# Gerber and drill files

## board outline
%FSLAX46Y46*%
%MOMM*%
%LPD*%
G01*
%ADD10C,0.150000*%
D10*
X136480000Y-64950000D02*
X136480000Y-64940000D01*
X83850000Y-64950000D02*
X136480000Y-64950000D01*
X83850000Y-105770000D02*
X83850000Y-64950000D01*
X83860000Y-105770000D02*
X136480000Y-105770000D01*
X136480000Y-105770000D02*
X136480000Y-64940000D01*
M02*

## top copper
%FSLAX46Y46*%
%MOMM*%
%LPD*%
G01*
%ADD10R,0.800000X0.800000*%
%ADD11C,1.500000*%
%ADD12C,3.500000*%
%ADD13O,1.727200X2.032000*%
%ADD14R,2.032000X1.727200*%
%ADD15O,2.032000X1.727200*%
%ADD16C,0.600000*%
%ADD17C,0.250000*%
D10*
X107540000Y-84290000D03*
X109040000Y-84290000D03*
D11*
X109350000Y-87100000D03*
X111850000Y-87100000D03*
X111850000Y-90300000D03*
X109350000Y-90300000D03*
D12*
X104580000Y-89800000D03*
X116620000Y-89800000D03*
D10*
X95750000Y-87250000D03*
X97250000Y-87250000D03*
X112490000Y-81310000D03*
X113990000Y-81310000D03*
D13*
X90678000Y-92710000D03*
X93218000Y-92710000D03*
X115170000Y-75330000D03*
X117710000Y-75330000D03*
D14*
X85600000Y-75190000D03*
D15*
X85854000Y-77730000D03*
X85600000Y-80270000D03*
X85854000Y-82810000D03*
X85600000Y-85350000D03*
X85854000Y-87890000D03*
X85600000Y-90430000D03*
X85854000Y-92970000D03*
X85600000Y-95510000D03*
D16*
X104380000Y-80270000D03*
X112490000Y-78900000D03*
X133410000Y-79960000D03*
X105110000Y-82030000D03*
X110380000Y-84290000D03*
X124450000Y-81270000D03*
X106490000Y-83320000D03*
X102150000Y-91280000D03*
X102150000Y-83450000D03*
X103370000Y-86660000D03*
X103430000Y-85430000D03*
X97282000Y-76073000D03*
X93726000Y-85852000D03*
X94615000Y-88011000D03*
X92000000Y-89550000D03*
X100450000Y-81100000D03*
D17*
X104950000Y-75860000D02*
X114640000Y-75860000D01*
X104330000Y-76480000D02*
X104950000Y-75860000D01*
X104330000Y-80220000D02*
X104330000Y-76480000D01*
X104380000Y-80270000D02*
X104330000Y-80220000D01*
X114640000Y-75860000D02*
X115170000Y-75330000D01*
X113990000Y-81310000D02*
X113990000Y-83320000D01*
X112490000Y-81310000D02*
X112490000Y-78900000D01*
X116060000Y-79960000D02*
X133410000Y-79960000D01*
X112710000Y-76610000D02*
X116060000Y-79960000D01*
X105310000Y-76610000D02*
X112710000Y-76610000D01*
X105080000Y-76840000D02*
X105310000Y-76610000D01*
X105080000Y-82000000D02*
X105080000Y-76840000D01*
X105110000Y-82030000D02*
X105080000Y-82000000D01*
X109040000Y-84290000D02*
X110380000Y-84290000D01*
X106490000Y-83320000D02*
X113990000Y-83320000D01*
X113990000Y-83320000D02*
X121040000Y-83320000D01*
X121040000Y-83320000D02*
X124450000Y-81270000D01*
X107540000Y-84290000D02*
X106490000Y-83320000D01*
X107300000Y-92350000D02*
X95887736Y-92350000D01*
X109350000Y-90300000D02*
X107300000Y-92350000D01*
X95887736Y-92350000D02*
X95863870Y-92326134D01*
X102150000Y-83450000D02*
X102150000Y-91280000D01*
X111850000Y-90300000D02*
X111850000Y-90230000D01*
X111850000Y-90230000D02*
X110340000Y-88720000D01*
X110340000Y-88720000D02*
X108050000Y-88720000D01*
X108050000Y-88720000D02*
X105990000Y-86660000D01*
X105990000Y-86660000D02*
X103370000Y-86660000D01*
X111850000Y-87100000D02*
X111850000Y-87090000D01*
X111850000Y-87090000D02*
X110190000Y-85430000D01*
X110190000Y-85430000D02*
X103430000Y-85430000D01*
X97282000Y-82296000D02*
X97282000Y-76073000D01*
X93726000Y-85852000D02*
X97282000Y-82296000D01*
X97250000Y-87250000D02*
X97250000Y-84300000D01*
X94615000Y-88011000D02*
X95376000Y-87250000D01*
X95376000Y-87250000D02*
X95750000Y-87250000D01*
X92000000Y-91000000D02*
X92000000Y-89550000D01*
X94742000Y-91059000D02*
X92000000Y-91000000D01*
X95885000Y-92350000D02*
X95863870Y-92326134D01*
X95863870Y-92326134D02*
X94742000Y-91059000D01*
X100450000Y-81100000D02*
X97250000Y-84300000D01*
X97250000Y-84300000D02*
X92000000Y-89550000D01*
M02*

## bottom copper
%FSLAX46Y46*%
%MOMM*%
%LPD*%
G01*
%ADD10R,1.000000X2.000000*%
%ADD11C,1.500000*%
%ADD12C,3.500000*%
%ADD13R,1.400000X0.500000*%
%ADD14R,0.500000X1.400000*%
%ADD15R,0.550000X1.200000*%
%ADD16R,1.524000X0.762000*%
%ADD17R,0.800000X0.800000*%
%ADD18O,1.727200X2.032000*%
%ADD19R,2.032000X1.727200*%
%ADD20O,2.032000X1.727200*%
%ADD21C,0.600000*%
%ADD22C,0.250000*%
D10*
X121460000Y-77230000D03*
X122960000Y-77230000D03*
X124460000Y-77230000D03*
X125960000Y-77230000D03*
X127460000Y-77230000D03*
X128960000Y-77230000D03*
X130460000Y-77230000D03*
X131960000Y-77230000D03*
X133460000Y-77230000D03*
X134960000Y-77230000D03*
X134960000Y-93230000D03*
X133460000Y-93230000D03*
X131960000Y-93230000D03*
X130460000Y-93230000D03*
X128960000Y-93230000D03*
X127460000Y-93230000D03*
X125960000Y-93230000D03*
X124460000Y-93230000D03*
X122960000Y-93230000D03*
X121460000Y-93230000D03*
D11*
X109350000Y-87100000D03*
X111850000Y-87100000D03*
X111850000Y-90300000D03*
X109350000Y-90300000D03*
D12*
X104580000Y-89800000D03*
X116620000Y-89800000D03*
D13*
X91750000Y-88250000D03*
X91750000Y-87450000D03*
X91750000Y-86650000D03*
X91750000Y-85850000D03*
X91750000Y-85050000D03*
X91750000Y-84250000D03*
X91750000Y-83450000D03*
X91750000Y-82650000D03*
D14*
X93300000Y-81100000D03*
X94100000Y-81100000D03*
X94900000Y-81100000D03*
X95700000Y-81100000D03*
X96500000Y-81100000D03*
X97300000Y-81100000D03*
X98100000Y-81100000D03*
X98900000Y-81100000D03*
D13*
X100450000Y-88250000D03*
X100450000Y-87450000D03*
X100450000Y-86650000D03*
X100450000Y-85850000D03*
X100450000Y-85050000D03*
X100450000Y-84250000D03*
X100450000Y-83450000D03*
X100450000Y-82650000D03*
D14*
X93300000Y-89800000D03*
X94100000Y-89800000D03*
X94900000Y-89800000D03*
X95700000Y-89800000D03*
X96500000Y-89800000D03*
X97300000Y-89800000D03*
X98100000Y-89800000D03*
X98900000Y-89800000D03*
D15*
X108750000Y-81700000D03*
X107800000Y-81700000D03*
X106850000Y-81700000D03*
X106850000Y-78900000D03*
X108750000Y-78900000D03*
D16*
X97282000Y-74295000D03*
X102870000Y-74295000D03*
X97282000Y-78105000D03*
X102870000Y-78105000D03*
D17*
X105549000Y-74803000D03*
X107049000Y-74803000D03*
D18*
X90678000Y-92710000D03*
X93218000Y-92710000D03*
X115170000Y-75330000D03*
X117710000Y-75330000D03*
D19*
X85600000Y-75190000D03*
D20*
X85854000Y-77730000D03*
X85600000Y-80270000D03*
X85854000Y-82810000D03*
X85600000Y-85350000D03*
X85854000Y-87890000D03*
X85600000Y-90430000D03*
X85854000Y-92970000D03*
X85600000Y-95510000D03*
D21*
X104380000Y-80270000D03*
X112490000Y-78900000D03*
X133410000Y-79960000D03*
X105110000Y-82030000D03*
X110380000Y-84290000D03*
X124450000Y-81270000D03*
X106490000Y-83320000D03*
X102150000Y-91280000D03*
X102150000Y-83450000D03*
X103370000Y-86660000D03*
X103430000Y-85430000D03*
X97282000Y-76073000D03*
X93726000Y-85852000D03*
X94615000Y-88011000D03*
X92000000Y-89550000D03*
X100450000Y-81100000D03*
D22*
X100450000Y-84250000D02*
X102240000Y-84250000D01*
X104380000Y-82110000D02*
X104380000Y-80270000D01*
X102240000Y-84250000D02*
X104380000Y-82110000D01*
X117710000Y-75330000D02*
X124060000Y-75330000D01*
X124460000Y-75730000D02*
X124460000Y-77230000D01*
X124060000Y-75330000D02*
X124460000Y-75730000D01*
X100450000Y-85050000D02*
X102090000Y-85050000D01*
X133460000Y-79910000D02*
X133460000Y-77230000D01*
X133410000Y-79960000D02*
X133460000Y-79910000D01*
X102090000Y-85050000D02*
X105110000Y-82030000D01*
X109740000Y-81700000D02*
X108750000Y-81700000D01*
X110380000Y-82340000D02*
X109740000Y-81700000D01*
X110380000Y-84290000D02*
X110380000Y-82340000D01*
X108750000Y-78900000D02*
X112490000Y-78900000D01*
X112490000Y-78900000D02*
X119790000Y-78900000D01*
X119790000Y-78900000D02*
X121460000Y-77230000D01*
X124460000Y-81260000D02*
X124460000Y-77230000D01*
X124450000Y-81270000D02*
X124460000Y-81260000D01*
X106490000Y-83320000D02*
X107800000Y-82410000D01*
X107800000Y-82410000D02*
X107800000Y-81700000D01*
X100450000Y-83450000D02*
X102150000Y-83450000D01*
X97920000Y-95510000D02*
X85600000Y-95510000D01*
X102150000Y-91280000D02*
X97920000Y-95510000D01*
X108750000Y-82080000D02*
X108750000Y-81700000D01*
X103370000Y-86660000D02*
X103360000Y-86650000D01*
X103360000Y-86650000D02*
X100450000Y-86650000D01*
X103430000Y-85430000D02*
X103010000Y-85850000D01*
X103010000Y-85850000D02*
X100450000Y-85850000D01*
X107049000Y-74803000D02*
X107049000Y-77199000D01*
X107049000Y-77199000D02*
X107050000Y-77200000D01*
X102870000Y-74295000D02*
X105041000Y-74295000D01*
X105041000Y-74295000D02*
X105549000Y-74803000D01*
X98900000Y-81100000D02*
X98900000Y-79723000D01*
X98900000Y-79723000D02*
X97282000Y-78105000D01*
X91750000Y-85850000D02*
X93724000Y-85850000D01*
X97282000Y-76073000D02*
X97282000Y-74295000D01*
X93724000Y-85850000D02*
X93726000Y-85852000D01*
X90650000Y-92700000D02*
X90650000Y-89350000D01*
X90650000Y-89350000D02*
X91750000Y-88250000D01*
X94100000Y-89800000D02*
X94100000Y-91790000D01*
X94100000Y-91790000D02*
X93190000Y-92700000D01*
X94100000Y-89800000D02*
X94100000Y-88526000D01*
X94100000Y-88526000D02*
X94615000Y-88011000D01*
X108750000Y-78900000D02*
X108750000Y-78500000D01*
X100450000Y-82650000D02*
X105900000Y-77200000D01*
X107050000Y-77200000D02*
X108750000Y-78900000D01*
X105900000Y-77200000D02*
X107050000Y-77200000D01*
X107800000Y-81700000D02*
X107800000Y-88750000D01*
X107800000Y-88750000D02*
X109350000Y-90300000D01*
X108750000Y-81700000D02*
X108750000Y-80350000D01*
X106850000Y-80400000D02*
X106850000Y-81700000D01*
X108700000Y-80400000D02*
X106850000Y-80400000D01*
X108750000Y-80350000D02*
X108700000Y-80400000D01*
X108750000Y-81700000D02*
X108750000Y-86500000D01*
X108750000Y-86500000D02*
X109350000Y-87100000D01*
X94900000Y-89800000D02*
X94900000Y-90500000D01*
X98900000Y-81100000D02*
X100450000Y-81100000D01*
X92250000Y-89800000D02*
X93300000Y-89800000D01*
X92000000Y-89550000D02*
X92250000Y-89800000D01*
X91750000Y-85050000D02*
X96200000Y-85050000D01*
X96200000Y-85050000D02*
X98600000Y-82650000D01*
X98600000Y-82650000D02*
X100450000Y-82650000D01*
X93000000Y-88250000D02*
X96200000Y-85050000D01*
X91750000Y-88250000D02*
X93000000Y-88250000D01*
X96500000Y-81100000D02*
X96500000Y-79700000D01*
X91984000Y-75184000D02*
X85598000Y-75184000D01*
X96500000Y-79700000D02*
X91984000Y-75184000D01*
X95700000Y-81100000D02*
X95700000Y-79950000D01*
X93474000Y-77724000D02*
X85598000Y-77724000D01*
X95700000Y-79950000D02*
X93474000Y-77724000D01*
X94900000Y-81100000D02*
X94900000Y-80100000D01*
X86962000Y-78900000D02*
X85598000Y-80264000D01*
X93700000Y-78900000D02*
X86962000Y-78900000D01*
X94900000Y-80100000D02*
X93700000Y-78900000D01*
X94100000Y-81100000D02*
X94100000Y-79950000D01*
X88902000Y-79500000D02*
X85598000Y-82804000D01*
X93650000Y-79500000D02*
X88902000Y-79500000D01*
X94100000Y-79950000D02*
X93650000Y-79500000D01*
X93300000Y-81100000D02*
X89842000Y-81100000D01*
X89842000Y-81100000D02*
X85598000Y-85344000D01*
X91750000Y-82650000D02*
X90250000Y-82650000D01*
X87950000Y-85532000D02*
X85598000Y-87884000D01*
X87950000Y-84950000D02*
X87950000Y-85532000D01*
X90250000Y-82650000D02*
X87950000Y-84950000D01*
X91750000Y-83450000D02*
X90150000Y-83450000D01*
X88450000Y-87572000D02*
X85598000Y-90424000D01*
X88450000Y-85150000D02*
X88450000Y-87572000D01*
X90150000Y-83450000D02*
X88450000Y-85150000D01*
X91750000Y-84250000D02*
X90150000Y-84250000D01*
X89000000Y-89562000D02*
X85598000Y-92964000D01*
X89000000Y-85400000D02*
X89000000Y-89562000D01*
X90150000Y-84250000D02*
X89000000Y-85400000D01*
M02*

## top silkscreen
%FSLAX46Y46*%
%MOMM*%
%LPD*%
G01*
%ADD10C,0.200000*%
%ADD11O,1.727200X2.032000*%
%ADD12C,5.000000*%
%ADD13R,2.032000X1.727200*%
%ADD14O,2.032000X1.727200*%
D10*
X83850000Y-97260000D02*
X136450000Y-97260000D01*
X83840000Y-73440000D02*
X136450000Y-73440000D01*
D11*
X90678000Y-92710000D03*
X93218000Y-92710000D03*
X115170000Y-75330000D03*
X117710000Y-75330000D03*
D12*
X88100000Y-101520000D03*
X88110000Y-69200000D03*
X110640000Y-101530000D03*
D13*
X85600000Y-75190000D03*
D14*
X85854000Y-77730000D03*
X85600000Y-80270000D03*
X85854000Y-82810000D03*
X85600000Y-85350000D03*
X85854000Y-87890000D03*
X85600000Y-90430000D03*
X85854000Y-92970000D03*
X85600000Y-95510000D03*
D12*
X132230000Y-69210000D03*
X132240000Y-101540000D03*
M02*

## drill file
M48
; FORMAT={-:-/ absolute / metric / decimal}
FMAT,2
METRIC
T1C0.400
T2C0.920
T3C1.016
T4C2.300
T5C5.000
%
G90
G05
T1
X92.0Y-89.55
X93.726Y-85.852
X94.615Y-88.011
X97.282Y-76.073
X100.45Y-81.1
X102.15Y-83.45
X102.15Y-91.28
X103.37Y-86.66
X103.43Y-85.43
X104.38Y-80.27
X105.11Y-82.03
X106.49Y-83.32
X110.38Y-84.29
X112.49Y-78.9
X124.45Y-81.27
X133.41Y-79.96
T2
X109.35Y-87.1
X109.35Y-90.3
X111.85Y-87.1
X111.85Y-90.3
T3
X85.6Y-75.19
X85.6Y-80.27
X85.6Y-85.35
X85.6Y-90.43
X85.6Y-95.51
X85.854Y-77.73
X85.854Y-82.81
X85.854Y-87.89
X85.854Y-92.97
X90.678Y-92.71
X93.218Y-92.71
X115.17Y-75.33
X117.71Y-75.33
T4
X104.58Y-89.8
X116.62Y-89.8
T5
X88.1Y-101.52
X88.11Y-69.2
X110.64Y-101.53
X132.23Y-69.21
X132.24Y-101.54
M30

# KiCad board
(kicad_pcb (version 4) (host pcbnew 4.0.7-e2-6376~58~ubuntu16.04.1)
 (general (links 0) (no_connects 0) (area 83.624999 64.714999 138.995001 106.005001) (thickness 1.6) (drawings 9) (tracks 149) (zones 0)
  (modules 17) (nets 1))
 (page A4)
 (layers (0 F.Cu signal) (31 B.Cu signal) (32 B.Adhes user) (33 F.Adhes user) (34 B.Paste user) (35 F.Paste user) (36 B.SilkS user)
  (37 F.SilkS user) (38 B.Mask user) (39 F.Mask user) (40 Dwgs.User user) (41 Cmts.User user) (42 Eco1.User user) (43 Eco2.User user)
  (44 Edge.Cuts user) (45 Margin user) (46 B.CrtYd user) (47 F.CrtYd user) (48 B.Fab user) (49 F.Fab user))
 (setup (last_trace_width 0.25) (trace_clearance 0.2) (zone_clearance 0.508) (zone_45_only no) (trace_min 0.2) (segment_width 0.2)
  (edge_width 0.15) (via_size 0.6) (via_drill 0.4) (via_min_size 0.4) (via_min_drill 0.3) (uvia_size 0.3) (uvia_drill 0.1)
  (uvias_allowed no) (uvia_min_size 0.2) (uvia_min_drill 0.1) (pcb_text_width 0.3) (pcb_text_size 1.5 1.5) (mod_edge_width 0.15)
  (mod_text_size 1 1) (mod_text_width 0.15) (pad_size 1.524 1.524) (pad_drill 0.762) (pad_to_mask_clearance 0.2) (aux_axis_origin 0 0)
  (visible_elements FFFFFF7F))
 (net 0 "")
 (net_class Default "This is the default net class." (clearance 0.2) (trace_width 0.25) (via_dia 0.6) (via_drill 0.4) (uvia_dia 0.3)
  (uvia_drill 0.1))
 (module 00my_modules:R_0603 (layer F.Cu) (at 108.29 84.29)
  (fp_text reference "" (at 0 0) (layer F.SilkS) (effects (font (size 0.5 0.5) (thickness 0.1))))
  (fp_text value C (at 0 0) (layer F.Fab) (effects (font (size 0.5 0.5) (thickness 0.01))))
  (pad 1 smd rect (at -0.75 0) (size 0.8 0.8) (layers F.Cu F.Paste F.Mask))
  (pad 2 smd rect (at 0.75 0) (size 0.8 0.8) (layers F.Cu F.Paste F.Mask)))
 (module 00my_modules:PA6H (layer B.Cu) (at 128.21 85.23 270)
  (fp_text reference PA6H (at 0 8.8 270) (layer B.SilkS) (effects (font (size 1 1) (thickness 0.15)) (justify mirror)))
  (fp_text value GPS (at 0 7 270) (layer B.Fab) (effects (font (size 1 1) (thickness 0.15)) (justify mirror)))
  (pad VCC smd rect (at -8 6.75 270) (size 2 1) (layers B.Cu B.Paste B.Mask))
  (pad 2 smd rect (at -8 5.25 270) (size 2 1) (layers B.Cu B.Paste B.Mask))
  (pad GND smd rect (at -8 3.75 270) (size 2 1) (layers B.Cu B.Paste B.Mask))
  (pad 4 smd rect (at -8 2.25 270) (size 2 1) (layers B.Cu B.Paste B.Mask))
  (pad 5 smd rect (at -8 0.75 270) (size 2 1) (layers B.Cu B.Paste B.Mask))
  (pad 6 smd rect (at -8 -0.75 270) (size 2 1) (layers B.Cu B.Paste B.Mask))
  (pad 7 smd rect (at -8 -2.25 270) (size 2 1) (layers B.Cu B.Paste B.Mask))
  (pad 8 smd rect (at -8 -3.75 270) (size 2 1) (layers B.Cu B.Paste B.Mask))
  (pad TX smd rect (at -8 -5.25 270) (size 2 1) (layers B.Cu B.Paste B.Mask))
  (pad RX smd rect (at -8 -6.75 270) (size 2 1) (layers B.Cu B.Paste B.Mask))
  (pad 11 smd rect (at 8 -6.75 270) (size 2 1) (layers B.Cu B.Paste B.Mask))
  (pad 12 smd rect (at 8 -5.25 270) (size 2 1) (layers B.Cu B.Paste B.Mask))
  (pad 13 smd rect (at 8 -3.75 270) (size 2 1) (layers B.Cu B.Paste B.Mask))
  (pad 14 smd rect (at 8 -2.25 270) (size 2 1) (layers B.Cu B.Paste B.Mask))
  (pad 15 smd rect (at 8 -0.75 270) (size 2 1) (layers B.Cu B.Paste B.Mask))
  (pad 16 smd rect (at 8 0.75 270) (size 2 1) (layers B.Cu B.Paste B.Mask))
  (pad 17 smd rect (at 8 2.25 270) (size 2 1) (layers B.Cu B.Paste B.Mask))
  (pad 18 smd rect (at 8 3.75 270) (size 2 1) (layers B.Cu B.Paste B.Mask))
  (pad 19 smd rect (at 8 5.25 270) (size 2 1) (layers B.Cu B.Paste B.Mask))
  (pad 20 smd rect (at 8 6.75 270) (size 2 1) (layers B.Cu B.Paste B.Mask)))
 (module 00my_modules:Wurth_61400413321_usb (layer B.Cu) (at 110.6 89.8 180)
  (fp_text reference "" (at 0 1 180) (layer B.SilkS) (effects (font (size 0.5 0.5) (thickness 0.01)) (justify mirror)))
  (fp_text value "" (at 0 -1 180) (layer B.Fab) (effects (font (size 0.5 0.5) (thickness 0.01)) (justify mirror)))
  (pad V thru_hole circle (at 1.25 2.7 180) (size 1.5 1.5) (drill 0.92) (layers *.Cu *.Mask B.SilkS))
  (pad - thru_hole circle (at -1.25 2.7 180) (size 1.5 1.5) (drill 0.92) (layers *.Cu *.Mask B.SilkS))
  (pad + thru_hole circle (at -1.25 -0.5 180) (size 1.5 1.5) (drill 0.92) (layers *.Cu *.Mask B.SilkS))
  (pad G thru_hole circle (at 1.25 -0.5 180) (size 1.5 1.5) (drill 0.92) (layers *.Cu *.Mask B.SilkS))
  (pad X thru_hole circle (at 6.02 0 180) (size 3.5 3.5) (drill 2.3) (layers *.Cu *.Mask B.SilkS))
  (pad X thru_hole circle (at -6.02 0 180) (size 3.5 3.5) (drill 2.3) (layers *.Cu *.Mask B.SilkS)))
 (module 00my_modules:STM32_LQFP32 (layer B.Cu) (at 96.1 85.45)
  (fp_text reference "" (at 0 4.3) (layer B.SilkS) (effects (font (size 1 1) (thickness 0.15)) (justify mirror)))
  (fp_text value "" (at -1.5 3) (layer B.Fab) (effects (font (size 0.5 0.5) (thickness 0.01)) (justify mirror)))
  (pad 3.3 smd rect (at -4.35 2.8) (size 1.4 0.5) (layers B.Cu B.Paste B.Mask))
  (pad PF0 smd rect (at -4.35 2) (size 1.4 0.5) (layers B.Cu B.Paste B.Mask))
  (pad PF1 smd rect (at -4.35 1.2) (size 1.4 0.5) (layers B.Cu B.Paste B.Mask))
  (pad RST smd rect (at -4.35 0.4) (size 1.4 0.5) (layers B.Cu B.Paste B.Mask))
  (pad 3.3 smd rect (at -4.35 -0.4) (size 1.4 0.5) (layers B.Cu B.Paste B.Mask))
  (pad PA0 smd rect (at -4.35 -1.2) (size 1.4 0.5) (layers B.Cu B.Paste B.Mask))
  (pad PA1 smd rect (at -4.35 -2) (size 1.4 0.5) (layers B.Cu B.Paste B.Mask))
  (pad PA2 smd rect (at -4.35 -2.8) (size 1.4 0.5) (layers B.Cu B.Paste B.Mask))
  (pad PA3 smd rect (at -2.8 -4.35 270) (size 1.4 0.5) (layers B.Cu B.Paste B.Mask))
  (pad PA4 smd rect (at -2 -4.35 270) (size 1.4 0.5) (layers B.Cu B.Paste B.Mask))
  (pad PA5 smd rect (at -1.2 -4.35 270) (size 1.4 0.5) (layers B.Cu B.Paste B.Mask))
  (pad PA6 smd rect (at -0.4 -4.35 270) (size 1.4 0.5) (layers B.Cu B.Paste B.Mask))
  (pad PA7 smd rect (at 0.4 -4.35 270) (size 1.4 0.5) (layers B.Cu B.Paste B.Mask))
  (pad PB0 smd rect (at 1.2 -4.35 270) (size 1.4 0.5) (layers B.Cu B.Paste B.Mask))
  (pad PB1 smd rect (at 2 -4.35 270) (size 1.4 0.5) (layers B.Cu B.Paste B.Mask))
  (pad GND smd rect (at 2.8 -4.35 270) (size 1.4 0.5) (layers B.Cu B.Paste B.Mask))
  (pad PA14 smd rect (at 4.35 2.8) (size 1.4 0.5) (layers B.Cu B.Paste B.Mask))
  (pad PA13 smd rect (at 4.35 2) (size 1.4 0.5) (layers B.Cu B.Paste B.Mask))
  (pad PA12 smd rect (at 4.35 1.2) (size 1.4 0.5) (layers B.Cu B.Paste B.Mask))
  (pad PA11 smd rect (at 4.35 0.4) (size 1.4 0.5) (layers B.Cu B.Paste B.Mask))
  (pad PA10 smd rect (at 4.35 -0.4) (size 1.4 0.5) (layers B.Cu B.Paste B.Mask))
  (pad PA9 smd rect (at 4.35 -1.2) (size 1.4 0.5) (layers B.Cu B.Paste B.Mask))
  (pad PA8 smd rect (at 4.35 -2) (size 1.4 0.5) (layers B.Cu B.Paste B.Mask))
  (pad 3.3 smd rect (at 4.35 -2.8) (size 1.4 0.5) (layers B.Cu B.Paste B.Mask))
  (pad GND smd rect (at -2.8 4.35 270) (size 1.4 0.5) (layers B.Cu B.Paste B.Mask))
  (pad BOOT smd rect (at -2 4.35 270) (size 1.4 0.5) (layers B.Cu B.Paste B.Mask))
  (pad PB7 smd rect (at -1.2 4.35 270) (size 1.4 0.5) (layers B.Cu B.Paste B.Mask))
  (pad PB6 smd rect (at -0.4 4.35 270) (size 1.4 0.5) (layers B.Cu B.Paste B.Mask))
  (pad PB5 smd rect (at 0.4 4.35 270) (size 1.4 0.5) (layers B.Cu B.Paste B.Mask))
  (pad PB4 smd rect (at 1.2 4.35 270) (size 1.4 0.5) (layers B.Cu B.Paste B.Mask))
  (pad PB3 smd rect (at 2 4.35 270) (size 1.4 0.5) (layers B.Cu B.Paste B.Mask))
  (pad PA15 smd rect (at 2.8 4.35 270) (size 1.4 0.5) (layers B.Cu B.Paste B.Mask)))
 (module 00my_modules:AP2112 (layer B.Cu) (at 107.8 80.3 90)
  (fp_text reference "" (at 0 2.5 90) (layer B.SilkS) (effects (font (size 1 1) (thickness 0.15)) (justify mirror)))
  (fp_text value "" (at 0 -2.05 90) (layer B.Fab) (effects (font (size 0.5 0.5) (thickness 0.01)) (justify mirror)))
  (pad VIN smd rect (at -1.4 0.95 90) (size 1.2 0.55) (layers B.Cu B.Paste B.Mask))
  (pad GND smd rect (at -1.4 0 90) (size 1.2 0.55) (layers B.Cu B.Paste B.Mask))
  (pad EN smd rect (at -1.4 -0.95 90) (size 1.2 0.55) (layers B.Cu B.Paste B.Mask))
  (pad NC smd rect (at 1.4 -0.95 90) (size 1.2 0.55) (layers B.Cu B.Paste B.Mask))
  (pad VOUT smd rect (at 1.4 0.95 90) (size 1.2 0.55) (layers B.Cu B.Paste B.Mask)))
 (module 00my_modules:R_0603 (layer F.Cu) (at 96.5 87.25)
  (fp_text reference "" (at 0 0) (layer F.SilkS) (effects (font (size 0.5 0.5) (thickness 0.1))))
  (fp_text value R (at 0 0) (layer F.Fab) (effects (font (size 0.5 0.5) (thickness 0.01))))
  (pad 1 smd rect (at -0.75 0) (size 0.8 0.8) (layers F.Cu F.Paste F.Mask))
  (pad 2 smd rect (at 0.75 0) (size 0.8 0.8) (layers F.Cu F.Paste F.Mask)))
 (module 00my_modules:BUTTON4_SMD (layer B.Cu) (at 100.076 76.2)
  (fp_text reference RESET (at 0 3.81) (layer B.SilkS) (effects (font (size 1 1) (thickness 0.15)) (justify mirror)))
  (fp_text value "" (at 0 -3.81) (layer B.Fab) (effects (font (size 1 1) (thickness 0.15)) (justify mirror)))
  (pad 1 smd rect (at -2.794 -1.905) (size 1.524 0.762) (layers B.Cu B.Paste B.Mask))
  (pad 2 smd rect (at 2.794 -1.905) (size 1.524 0.762) (layers B.Cu B.Paste B.Mask))
  (pad 3 smd rect (at -2.794 1.905) (size 1.524 0.762) (layers B.Cu B.Paste B.Mask))
  (pad 4 smd rect (at 2.794 1.905) (size 1.524 0.762) (layers B.Cu B.Paste B.Mask)))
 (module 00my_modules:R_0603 (layer B.Cu) (at 106.299 74.803)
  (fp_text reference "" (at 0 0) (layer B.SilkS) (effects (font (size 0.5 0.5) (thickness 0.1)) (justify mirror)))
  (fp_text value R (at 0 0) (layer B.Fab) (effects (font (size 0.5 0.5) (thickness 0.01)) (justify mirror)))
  (pad 1 smd rect (at -0.75 0) (size 0.8 0.8) (layers B.Cu B.Paste B.Mask))
  (pad 2 smd rect (at 0.75 0) (size 0.8 0.8) (layers B.Cu B.Paste B.Mask)))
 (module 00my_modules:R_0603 (layer F.Cu) (at 113.24 81.31)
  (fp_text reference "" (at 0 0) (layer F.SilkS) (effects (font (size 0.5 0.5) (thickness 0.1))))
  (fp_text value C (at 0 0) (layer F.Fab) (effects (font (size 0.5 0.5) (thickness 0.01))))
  (pad 1 smd rect (at -0.75 0) (size 0.8 0.8) (layers F.Cu F.Paste F.Mask))
  (pad 2 smd rect (at 0.75 0) (size 0.8 0.8) (layers F.Cu F.Paste F.Mask)))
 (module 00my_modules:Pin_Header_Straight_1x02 (layer F.Cu) (at 90.678 92.71 90)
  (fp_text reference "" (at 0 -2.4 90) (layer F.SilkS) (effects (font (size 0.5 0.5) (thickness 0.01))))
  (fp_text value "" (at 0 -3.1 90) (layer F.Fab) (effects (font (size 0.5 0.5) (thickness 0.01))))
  (pad 1 thru_hole oval (at 0 0 90) (size 2.032 1.7272) (drill 1.016) (layers *.Cu *.Mask F.SilkS))
  (pad 2 thru_hole oval (at 0 2.54 90) (size 2.032 1.7272) (drill 1.016) (layers *.Cu *.Mask F.SilkS)))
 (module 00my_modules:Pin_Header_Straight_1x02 (layer F.Cu) (at 115.17 75.33 90)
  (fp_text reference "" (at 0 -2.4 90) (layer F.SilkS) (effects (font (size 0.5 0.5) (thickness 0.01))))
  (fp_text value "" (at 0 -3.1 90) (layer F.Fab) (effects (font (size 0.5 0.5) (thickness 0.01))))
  (pad 1 thru_hole oval (at 0 0 90) (size 2.032 1.7272) (drill 1.016) (layers *.Cu *.Mask F.SilkS))
  (pad 2 thru_hole oval (at 0 2.54 90) (size 2.032 1.7272) (drill 1.016) (layers *.Cu *.Mask F.SilkS)))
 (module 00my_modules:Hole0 (layer F.Cu) (at 88.1 101.52)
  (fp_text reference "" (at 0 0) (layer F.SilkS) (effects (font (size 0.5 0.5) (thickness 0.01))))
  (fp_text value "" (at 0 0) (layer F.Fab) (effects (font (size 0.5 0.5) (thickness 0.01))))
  (pad "" np_thru_hole circle (at 0 0) (size 5 5) (drill 5) (layers *.Cu *.Mask F.SilkS)))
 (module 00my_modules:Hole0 (layer F.Cu) (at 88.11 69.2)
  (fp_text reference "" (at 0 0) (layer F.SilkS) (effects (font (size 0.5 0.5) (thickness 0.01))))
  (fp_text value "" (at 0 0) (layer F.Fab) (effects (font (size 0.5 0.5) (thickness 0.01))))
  (pad "" np_thru_hole circle (at 0 0) (size 5 5) (drill 5) (layers *.Cu *.Mask F.SilkS)))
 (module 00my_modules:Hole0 (layer F.Cu) (at 110.64 101.53)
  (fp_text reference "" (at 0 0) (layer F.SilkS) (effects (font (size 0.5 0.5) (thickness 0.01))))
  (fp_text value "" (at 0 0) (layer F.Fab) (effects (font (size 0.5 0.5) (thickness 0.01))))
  (pad "" np_thru_hole circle (at 0 0) (size 5 5) (drill 5) (layers *.Cu *.Mask F.SilkS)))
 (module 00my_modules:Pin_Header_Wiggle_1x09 (layer F.Cu) (at 85.6 75.19)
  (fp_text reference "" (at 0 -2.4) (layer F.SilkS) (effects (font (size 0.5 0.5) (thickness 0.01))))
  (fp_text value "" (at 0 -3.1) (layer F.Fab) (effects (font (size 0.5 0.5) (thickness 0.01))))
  (pad 1 thru_hole rect (at 0 0) (size 2.032 1.7272) (drill 1.016) (layers *.Cu *.Mask F.SilkS))
  (pad 2 thru_hole oval (at 0.254 2.54) (size 2.032 1.7272) (drill 1.016) (layers *.Cu *.Mask F.SilkS))
  (pad 3 thru_hole oval (at 0 5.08) (size 2.032 1.7272) (drill 1.016) (layers *.Cu *.Mask F.SilkS))
  (pad 4 thru_hole oval (at 0.254 7.62) (size 2.032 1.7272) (drill 1.016) (layers *.Cu *.Mask F.SilkS))
  (pad 5 thru_hole oval (at 0 10.16) (size 2.032 1.7272) (drill 1.016) (layers *.Cu *.Mask F.SilkS))
  (pad 6 thru_hole oval (at 0.254 12.7) (size 2.032 1.7272) (drill 1.016) (layers *.Cu *.Mask F.SilkS))
  (pad 7 thru_hole oval (at 0 15.24) (size 2.032 1.7272) (drill 1.016) (layers *.Cu *.Mask F.SilkS))
  (pad 8 thru_hole oval (at 0.254 17.78) (size 2.032 1.7272) (drill 1.016) (layers *.Cu *.Mask F.SilkS))
  (pad 9 thru_hole oval (at 0 20.32) (size 2.032 1.7272) (drill 1.016) (layers *.Cu *.Mask F.SilkS)))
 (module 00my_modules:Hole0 (layer F.Cu) (at 132.23 69.21)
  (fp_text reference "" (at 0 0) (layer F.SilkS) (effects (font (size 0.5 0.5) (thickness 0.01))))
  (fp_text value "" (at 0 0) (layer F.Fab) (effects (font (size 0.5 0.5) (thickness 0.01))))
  (pad "" np_thru_hole circle (at 0 0) (size 5 5) (drill 5) (layers *.Cu *.Mask F.SilkS)))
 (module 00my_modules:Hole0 (layer F.Cu) (at 132.24 101.54)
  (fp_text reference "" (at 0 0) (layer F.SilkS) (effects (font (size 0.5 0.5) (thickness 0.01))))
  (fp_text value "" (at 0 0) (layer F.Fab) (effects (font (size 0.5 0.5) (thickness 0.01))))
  (pad "" np_thru_hole circle (at 0 0) (size 5 5) (drill 5) (layers *.Cu *.Mask F.SilkS)))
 (gr_line (start 83.85 97.26) (end 136.45 97.26) (angle 90) (layer F.SilkS) (width 0.2))
 (gr_line (start 83.84 73.44) (end 136.45 73.44) (angle 90) (layer F.SilkS) (width 0.2))
 (gr_line (start 136.48 64.95) (end 136.48 64.94) (angle 90) (layer Edge.Cuts) (width 0.15))
 (gr_line (start 83.85 64.95) (end 136.48 64.95) (angle 90) (layer Edge.Cuts) (width 0.15))
 (gr_line (start 83.85 105.77) (end 83.85 64.95) (angle 90) (layer Edge.Cuts) (width 0.15))
 (gr_line (start 83.86 105.77) (end 136.48 105.77) (angle 90) (layer Edge.Cuts) (width 0.15))
 (gr_line (start 136.48 105.77) (end 136.48 64.94) (angle 90) (layer Edge.Cuts) (width 0.15))
 (segment (start 100.45 84.25) (end 102.24 84.25) (width 0.25) (layer B.Cu) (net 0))
 (segment (start 104.95 75.86) (end 114.64 75.86) (width 0.25) (layer F.Cu) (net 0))
 (segment (start 104.33 76.48) (end 104.95 75.86) (width 0.25) (layer F.Cu) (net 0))
 (segment (start 104.33 80.22) (end 104.33 76.48) (width 0.25) (layer F.Cu) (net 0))
 (segment (start 104.38 80.27) (end 104.33 80.22) (width 0.25) (layer F.Cu) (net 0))
 (via (at 104.38 80.27) (size 0.6) (drill 0.4) (layers F.Cu B.Cu) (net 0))
 (segment (start 104.38 82.11) (end 104.38 80.27) (width 0.25) (layer B.Cu) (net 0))
 (segment (start 102.24 84.25) (end 104.38 82.11) (width 0.25) (layer B.Cu) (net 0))
 (segment (start 114.64 75.86) (end 115.17 75.33) (width 0.25) (layer F.Cu) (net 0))
 (segment (start 117.71 75.33) (end 124.06 75.33) (width 0.25) (layer B.Cu) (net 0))
 (segment (start 124.46 75.73) (end 124.46 77.23) (width 0.25) (layer B.Cu) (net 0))
 (segment (start 124.06 75.33) (end 124.46 75.73) (width 0.25) (layer B.Cu) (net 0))
 (segment (start 113.99 81.31) (end 113.99 83.32) (width 0.25) (layer F.Cu) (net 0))
 (segment (start 112.49 81.31) (end 112.49 78.9) (width 0.25) (layer F.Cu) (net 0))
 (via (at 112.49 78.9) (size 0.6) (drill 0.4) (layers F.Cu B.Cu) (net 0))
 (segment (start 100.45 85.05) (end 102.09 85.05) (width 0.25) (layer B.Cu) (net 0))
 (segment (start 133.46 79.91) (end 133.46 77.23) (width 0.25) (layer B.Cu) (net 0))
 (segment (start 133.41 79.96) (end 133.46 79.91) (width 0.25) (layer B.Cu) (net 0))
 (via (at 133.41 79.96) (size 0.6) (drill 0.4) (layers F.Cu B.Cu) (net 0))
 (segment (start 116.06 79.96) (end 133.41 79.96) (width 0.25) (layer F.Cu) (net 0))
 (segment (start 112.71 76.61) (end 116.06 79.96) (width 0.25) (layer F.Cu) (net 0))
 (segment (start 105.31 76.61) (end 112.71 76.61) (width 0.25) (layer F.Cu) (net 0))
 (segment (start 105.08 76.84) (end 105.31 76.61) (width 0.25) (layer F.Cu) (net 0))
 (segment (start 105.08 82) (end 105.08 76.84) (width 0.25) (layer F.Cu) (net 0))
 (segment (start 105.11 82.03) (end 105.08 82) (width 0.25) (layer F.Cu) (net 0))
 (via (at 105.11 82.03) (size 0.6) (drill 0.4) (layers F.Cu B.Cu) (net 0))
 (segment (start 102.09 85.05) (end 105.11 82.03) (width 0.25) (layer B.Cu) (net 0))
 (segment (start 109.04 84.29) (end 110.38 84.29) (width 0.25) (layer F.Cu) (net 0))
 (segment (start 109.74 81.7) (end 108.75 81.7) (width 0.25) (layer B.Cu) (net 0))
 (segment (start 110.38 82.34) (end 109.74 81.7) (width 0.25) (layer B.Cu) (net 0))
 (segment (start 110.38 84.29) (end 110.38 82.34) (width 0.25) (layer B.Cu) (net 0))
 (via (at 110.38 84.29) (size 0.6) (drill 0.4) (layers F.Cu B.Cu) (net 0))
 (segment (start 108.75 78.9) (end 112.49 78.9) (width 0.25) (layer B.Cu) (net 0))
 (segment (start 112.49 78.9) (end 119.79 78.9) (width 0.25) (layer B.Cu) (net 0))
 (segment (start 119.79 78.9) (end 121.46 77.23) (width 0.25) (layer B.Cu) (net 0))
 (segment (start 106.49 83.32) (end 113.99 83.32) (width 0.25) (layer F.Cu) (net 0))
 (segment (start 113.99 83.32) (end 121.04 83.32) (width 0.25) (layer F.Cu) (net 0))
 (segment (start 124.46 81.26) (end 124.46 77.23) (width 0.25) (layer B.Cu) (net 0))
 (segment (start 124.45 81.27) (end 124.46 81.26) (width 0.25) (layer B.Cu) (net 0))
 (via (at 124.45 81.27) (size 0.6) (drill 0.4) (layers F.Cu B.Cu) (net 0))
 (segment (start 121.04 83.32) (end 124.45 81.27) (width 0.25) (layer F.Cu) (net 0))
 (segment (start 107.54 84.29) (end 106.49 83.32) (width 0.25) (layer F.Cu) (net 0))
 (via (at 106.49 83.32) (size 0.6) (drill 0.4) (layers F.Cu B.Cu) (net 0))
 (segment (start 106.49 83.32) (end 107.8 82.41) (width 0.25) (layer B.Cu) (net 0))
 (segment (start 107.8 82.41) (end 107.8 81.7) (width 0.25) (layer B.Cu) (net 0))
 (segment (start 107.3 92.35) (end 95.887736 92.35) (width 0.25) (layer F.Cu) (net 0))
 (segment (start 109.35 90.3) (end 107.3 92.35) (width 0.25) (layer F.Cu) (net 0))
 (segment (start 95.887736 92.35) (end 95.86387 92.326134) (width 0.25) (layer F.Cu) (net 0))
 (segment (start 100.45 83.45) (end 102.15 83.45) (width 0.25) (layer B.Cu) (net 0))
 (segment (start 97.92 95.51) (end 85.6 95.51) (width 0.25) (layer B.Cu) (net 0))
 (segment (start 102.15 91.28) (end 97.92 95.51) (width 0.25) (layer B.Cu) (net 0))
 (via (at 102.15 91.28) (size 0.6) (drill 0.4) (layers F.Cu B.Cu) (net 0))
 (segment (start 102.15 83.45) (end 102.15 91.28) (width 0.25) (layer F.Cu) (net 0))
 (via (at 102.15 83.45) (size 0.6) (drill 0.4) (layers F.Cu B.Cu) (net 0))
 (segment (start 108.75 82.08) (end 108.75 81.7) (width 0.25) (layer B.Cu) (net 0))
 (segment (start 111.85 90.3) (end 111.85 90.23) (width 0.25) (layer F.Cu) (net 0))
 (segment (start 111.85 90.23) (end 110.34 88.72) (width 0.25) (layer F.Cu) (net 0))
 (segment (start 110.34 88.72) (end 108.05 88.72) (width 0.25) (layer F.Cu) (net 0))
 (segment (start 108.05 88.72) (end 105.99 86.66) (width 0.25) (layer F.Cu) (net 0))
 (segment (start 105.99 86.66) (end 103.37 86.66) (width 0.25) (layer F.Cu) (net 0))
 (via (at 103.37 86.66) (size 0.6) (drill 0.4) (layers F.Cu B.Cu) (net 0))
 (segment (start 103.37 86.66) (end 103.36 86.65) (width 0.25) (layer B.Cu) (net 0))
 (segment (start 103.36 86.65) (end 100.45 86.65) (width 0.25) (layer B.Cu) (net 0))
 (segment (start 111.85 87.1) (end 111.85 87.09) (width 0.25) (layer F.Cu) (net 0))
 (segment (start 111.85 87.09) (end 110.19 85.43) (width 0.25) (layer F.Cu) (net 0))
 (segment (start 110.19 85.43) (end 103.43 85.43) (width 0.25) (layer F.Cu) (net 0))
 (via (at 103.43 85.43) (size 0.6) (drill 0.4) (layers F.Cu B.Cu) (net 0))
 (segment (start 103.43 85.43) (end 103.01 85.85) (width 0.25) (layer B.Cu) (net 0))
 (segment (start 103.01 85.85) (end 100.45 85.85) (width 0.25) (layer B.Cu) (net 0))
 (segment (start 107.049 74.803) (end 107.049 77.199) (width 0.25) (layer B.Cu) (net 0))
 (segment (start 107.049 77.199) (end 107.05 77.2) (width 0.25) (layer B.Cu) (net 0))
 (segment (start 102.87 74.295) (end 105.041 74.295) (width 0.25) (layer B.Cu) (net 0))
 (segment (start 105.041 74.295) (end 105.549 74.803) (width 0.25) (layer B.Cu) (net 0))
 (segment (start 98.9 81.1) (end 98.9 79.723) (width 0.25) (layer B.Cu) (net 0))
 (segment (start 98.9 79.723) (end 97.282 78.105) (width 0.25) (layer B.Cu) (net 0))
 (segment (start 91.75 85.85) (end 93.724 85.85) (width 0.25) (layer B.Cu) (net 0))
 (segment (start 97.282 76.073) (end 97.282 74.295) (width 0.25) (layer B.Cu) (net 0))
 (via (at 97.282 76.073) (size 0.6) (drill 0.4) (layers F.Cu B.Cu) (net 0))
 (segment (start 97.282 82.296) (end 97.282 76.073) (width 0.25) (layer F.Cu) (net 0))
 (segment (start 93.726 85.852) (end 97.282 82.296) (width 0.25) (layer F.Cu) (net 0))
 (via (at 93.726 85.852) (size 0.6) (drill 0.4) (layers F.Cu B.Cu) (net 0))
 (segment (start 93.724 85.85) (end 93.726 85.852) (width 0.25) (layer B.Cu) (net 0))
 (segment (start 90.65 92.7) (end 90.65 89.35) (width 0.25) (layer B.Cu) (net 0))
 (segment (start 90.65 89.35) (end 91.75 88.25) (width 0.25) (layer B.Cu) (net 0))
 (segment (start 94.1 89.8) (end 94.1 91.79) (width 0.25) (layer B.Cu) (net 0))
 (segment (start 94.1 91.79) (end 93.19 92.7) (width 0.25) (layer B.Cu) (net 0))
 (segment (start 97.25 87.25) (end 97.25 84.3) (width 0.25) (layer F.Cu) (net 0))
 (segment (start 94.1 89.8) (end 94.1 88.526) (width 0.25) (layer B.Cu) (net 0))
 (segment (start 94.615 88.011) (end 95.376 87.25) (width 0.25) (layer F.Cu) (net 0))
 (via (at 94.615 88.011) (size 0.6) (drill 0.4) (layers F.Cu B.Cu) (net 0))
 (segment (start 94.1 88.526) (end 94.615 88.011) (width 0.25) (layer B.Cu) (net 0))
 (segment (start 95.376 87.25) (end 95.75 87.25) (width 0.25) (layer F.Cu) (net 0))
 (segment (start 108.75 78.9) (end 108.75 78.5) (width 0.25) (layer B.Cu) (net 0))
 (segment (start 100.45 82.65) (end 105.9 77.2) (width 0.25) (layer B.Cu) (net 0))
 (segment (start 107.05 77.2) (end 108.75 78.9) (width 0.25) (layer B.Cu) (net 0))
 (segment (start 105.9 77.2) (end 107.05 77.2) (width 0.25) (layer B.Cu) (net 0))
 (segment (start 107.8 81.7) (end 107.8 88.75) (width 0.25) (layer B.Cu) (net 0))
 (segment (start 107.8 88.75) (end 109.35 90.3) (width 0.25) (layer B.Cu) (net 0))
 (segment (start 108.75 81.7) (end 108.75 80.35) (width 0.25) (layer B.Cu) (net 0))
 (segment (start 106.85 80.4) (end 106.85 81.7) (width 0.25) (layer B.Cu) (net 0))
 (segment (start 108.7 80.4) (end 106.85 80.4) (width 0.25) (layer B.Cu) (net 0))
 (segment (start 108.75 80.35) (end 108.7 80.4) (width 0.25) (layer B.Cu) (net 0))
 (segment (start 108.75 81.7) (end 108.75 86.5) (width 0.25) (layer B.Cu) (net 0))
 (segment (start 108.75 86.5) (end 109.35 87.1) (width 0.25) (layer B.Cu) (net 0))
 (segment (start 92 91) (end 92 89.55) (width 0.25) (layer F.Cu) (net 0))
 (segment (start 94.742 91.059) (end 92 91) (width 0.25) (layer F.Cu) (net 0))
 (segment (start 95.885 92.35) (end 95.86387 92.326134) (width 0.25) (layer F.Cu) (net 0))
 (segment (start 95.86387 92.326134) (end 94.742 91.059) (width 0.25) (layer F.Cu) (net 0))
 (segment (start 94.9 89.8) (end 94.9 90.5) (width 0.25) (layer B.Cu) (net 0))
 (segment (start 98.9 81.1) (end 100.45 81.1) (width 0.25) (layer B.Cu) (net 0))
 (segment (start 92.25 89.8) (end 93.3 89.8) (width 0.25) (layer B.Cu) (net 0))
 (segment (start 92 89.55) (end 92.25 89.8) (width 0.25) (layer B.Cu) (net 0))
 (via (at 92 89.55) (size 0.6) (drill 0.4) (layers F.Cu B.Cu) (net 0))
 (segment (start 100.45 81.1) (end 97.25 84.3) (width 0.25) (layer F.Cu) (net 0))
 (segment (start 97.25 84.3) (end 92 89.55) (width 0.25) (layer F.Cu) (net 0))
 (via (at 100.45 81.1) (size 0.6) (drill 0.4) (layers F.Cu B.Cu) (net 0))
 (segment (start 91.75 85.05) (end 96.2 85.05) (width 0.25) (layer B.Cu) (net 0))
 (segment (start 96.2 85.05) (end 98.6 82.65) (width 0.25) (layer B.Cu) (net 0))
 (segment (start 98.6 82.65) (end 100.45 82.65) (width 0.25) (layer B.Cu) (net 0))
 (segment (start 93 88.25) (end 96.2 85.05) (width 0.25) (layer B.Cu) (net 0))
 (segment (start 91.75 88.25) (end 93 88.25) (width 0.25) (layer B.Cu) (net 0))
 (segment (start 96.5 81.1) (end 96.5 79.7) (width 0.25) (layer B.Cu) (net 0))
 (segment (start 91.984 75.184) (end 85.598 75.184) (width 0.25) (layer B.Cu) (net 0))
 (segment (start 96.5 79.7) (end 91.984 75.184) (width 0.25) (layer B.Cu) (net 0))
 (segment (start 95.7 81.1) (end 95.7 79.95) (width 0.25) (layer B.Cu) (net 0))
 (segment (start 93.474 77.724) (end 85.598 77.724) (width 0.25) (layer B.Cu) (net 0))
 (segment (start 95.7 79.95) (end 93.474 77.724) (width 0.25) (layer B.Cu) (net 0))
 (segment (start 94.9 81.1) (end 94.9 80.1) (width 0.25) (layer B.Cu) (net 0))
 (segment (start 86.962 78.9) (end 85.598 80.264) (width 0.25) (layer B.Cu) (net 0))
 (segment (start 93.7 78.9) (end 86.962 78.9) (width 0.25) (layer B.Cu) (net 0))
 (segment (start 94.9 80.1) (end 93.7 78.9) (width 0.25) (layer B.Cu) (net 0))
 (segment (start 94.1 81.1) (end 94.1 79.95) (width 0.25) (layer B.Cu) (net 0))
 (segment (start 88.902 79.5) (end 85.598 82.804) (width 0.25) (layer B.Cu) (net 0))
 (segment (start 93.65 79.5) (end 88.902 79.5) (width 0.25) (layer B.Cu) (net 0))
 (segment (start 94.1 79.95) (end 93.65 79.5) (width 0.25) (layer B.Cu) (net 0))
 (segment (start 93.3 81.1) (end 89.842 81.1) (width 0.25) (layer B.Cu) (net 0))
 (segment (start 89.842 81.1) (end 85.598 85.344) (width 0.25) (layer B.Cu) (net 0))
 (segment (start 91.75 82.65) (end 90.25 82.65) (width 0.25) (layer B.Cu) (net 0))
 (segment (start 87.95 85.532) (end 85.598 87.884) (width 0.25) (layer B.Cu) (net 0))
 (segment (start 87.95 84.95) (end 87.95 85.532) (width 0.25) (layer B.Cu) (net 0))
 (segment (start 90.25 82.65) (end 87.95 84.95) (width 0.25) (layer B.Cu) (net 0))
 (segment (start 91.75 83.45) (end 90.15 83.45) (width 0.25) (layer B.Cu) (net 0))
 (segment (start 88.45 87.572) (end 85.598 90.424) (width 0.25) (layer B.Cu) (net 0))
 (segment (start 88.45 85.15) (end 88.45 87.572) (width 0.25) (layer B.Cu) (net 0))
 (segment (start 90.15 83.45) (end 88.45 85.15) (width 0.25) (layer B.Cu) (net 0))
 (segment (start 91.75 84.25) (end 90.15 84.25) (width 0.25) (layer B.Cu) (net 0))
 (segment (start 89 89.562) (end 85.598 92.964) (width 0.25) (layer B.Cu) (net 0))
 (segment (start 89 85.4) (end 89 89.562) (width 0.25) (layer B.Cu) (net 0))
 (segment (start 90.15 84.25) (end 89 85.4) (width 0.25) (layer B.Cu) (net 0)))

